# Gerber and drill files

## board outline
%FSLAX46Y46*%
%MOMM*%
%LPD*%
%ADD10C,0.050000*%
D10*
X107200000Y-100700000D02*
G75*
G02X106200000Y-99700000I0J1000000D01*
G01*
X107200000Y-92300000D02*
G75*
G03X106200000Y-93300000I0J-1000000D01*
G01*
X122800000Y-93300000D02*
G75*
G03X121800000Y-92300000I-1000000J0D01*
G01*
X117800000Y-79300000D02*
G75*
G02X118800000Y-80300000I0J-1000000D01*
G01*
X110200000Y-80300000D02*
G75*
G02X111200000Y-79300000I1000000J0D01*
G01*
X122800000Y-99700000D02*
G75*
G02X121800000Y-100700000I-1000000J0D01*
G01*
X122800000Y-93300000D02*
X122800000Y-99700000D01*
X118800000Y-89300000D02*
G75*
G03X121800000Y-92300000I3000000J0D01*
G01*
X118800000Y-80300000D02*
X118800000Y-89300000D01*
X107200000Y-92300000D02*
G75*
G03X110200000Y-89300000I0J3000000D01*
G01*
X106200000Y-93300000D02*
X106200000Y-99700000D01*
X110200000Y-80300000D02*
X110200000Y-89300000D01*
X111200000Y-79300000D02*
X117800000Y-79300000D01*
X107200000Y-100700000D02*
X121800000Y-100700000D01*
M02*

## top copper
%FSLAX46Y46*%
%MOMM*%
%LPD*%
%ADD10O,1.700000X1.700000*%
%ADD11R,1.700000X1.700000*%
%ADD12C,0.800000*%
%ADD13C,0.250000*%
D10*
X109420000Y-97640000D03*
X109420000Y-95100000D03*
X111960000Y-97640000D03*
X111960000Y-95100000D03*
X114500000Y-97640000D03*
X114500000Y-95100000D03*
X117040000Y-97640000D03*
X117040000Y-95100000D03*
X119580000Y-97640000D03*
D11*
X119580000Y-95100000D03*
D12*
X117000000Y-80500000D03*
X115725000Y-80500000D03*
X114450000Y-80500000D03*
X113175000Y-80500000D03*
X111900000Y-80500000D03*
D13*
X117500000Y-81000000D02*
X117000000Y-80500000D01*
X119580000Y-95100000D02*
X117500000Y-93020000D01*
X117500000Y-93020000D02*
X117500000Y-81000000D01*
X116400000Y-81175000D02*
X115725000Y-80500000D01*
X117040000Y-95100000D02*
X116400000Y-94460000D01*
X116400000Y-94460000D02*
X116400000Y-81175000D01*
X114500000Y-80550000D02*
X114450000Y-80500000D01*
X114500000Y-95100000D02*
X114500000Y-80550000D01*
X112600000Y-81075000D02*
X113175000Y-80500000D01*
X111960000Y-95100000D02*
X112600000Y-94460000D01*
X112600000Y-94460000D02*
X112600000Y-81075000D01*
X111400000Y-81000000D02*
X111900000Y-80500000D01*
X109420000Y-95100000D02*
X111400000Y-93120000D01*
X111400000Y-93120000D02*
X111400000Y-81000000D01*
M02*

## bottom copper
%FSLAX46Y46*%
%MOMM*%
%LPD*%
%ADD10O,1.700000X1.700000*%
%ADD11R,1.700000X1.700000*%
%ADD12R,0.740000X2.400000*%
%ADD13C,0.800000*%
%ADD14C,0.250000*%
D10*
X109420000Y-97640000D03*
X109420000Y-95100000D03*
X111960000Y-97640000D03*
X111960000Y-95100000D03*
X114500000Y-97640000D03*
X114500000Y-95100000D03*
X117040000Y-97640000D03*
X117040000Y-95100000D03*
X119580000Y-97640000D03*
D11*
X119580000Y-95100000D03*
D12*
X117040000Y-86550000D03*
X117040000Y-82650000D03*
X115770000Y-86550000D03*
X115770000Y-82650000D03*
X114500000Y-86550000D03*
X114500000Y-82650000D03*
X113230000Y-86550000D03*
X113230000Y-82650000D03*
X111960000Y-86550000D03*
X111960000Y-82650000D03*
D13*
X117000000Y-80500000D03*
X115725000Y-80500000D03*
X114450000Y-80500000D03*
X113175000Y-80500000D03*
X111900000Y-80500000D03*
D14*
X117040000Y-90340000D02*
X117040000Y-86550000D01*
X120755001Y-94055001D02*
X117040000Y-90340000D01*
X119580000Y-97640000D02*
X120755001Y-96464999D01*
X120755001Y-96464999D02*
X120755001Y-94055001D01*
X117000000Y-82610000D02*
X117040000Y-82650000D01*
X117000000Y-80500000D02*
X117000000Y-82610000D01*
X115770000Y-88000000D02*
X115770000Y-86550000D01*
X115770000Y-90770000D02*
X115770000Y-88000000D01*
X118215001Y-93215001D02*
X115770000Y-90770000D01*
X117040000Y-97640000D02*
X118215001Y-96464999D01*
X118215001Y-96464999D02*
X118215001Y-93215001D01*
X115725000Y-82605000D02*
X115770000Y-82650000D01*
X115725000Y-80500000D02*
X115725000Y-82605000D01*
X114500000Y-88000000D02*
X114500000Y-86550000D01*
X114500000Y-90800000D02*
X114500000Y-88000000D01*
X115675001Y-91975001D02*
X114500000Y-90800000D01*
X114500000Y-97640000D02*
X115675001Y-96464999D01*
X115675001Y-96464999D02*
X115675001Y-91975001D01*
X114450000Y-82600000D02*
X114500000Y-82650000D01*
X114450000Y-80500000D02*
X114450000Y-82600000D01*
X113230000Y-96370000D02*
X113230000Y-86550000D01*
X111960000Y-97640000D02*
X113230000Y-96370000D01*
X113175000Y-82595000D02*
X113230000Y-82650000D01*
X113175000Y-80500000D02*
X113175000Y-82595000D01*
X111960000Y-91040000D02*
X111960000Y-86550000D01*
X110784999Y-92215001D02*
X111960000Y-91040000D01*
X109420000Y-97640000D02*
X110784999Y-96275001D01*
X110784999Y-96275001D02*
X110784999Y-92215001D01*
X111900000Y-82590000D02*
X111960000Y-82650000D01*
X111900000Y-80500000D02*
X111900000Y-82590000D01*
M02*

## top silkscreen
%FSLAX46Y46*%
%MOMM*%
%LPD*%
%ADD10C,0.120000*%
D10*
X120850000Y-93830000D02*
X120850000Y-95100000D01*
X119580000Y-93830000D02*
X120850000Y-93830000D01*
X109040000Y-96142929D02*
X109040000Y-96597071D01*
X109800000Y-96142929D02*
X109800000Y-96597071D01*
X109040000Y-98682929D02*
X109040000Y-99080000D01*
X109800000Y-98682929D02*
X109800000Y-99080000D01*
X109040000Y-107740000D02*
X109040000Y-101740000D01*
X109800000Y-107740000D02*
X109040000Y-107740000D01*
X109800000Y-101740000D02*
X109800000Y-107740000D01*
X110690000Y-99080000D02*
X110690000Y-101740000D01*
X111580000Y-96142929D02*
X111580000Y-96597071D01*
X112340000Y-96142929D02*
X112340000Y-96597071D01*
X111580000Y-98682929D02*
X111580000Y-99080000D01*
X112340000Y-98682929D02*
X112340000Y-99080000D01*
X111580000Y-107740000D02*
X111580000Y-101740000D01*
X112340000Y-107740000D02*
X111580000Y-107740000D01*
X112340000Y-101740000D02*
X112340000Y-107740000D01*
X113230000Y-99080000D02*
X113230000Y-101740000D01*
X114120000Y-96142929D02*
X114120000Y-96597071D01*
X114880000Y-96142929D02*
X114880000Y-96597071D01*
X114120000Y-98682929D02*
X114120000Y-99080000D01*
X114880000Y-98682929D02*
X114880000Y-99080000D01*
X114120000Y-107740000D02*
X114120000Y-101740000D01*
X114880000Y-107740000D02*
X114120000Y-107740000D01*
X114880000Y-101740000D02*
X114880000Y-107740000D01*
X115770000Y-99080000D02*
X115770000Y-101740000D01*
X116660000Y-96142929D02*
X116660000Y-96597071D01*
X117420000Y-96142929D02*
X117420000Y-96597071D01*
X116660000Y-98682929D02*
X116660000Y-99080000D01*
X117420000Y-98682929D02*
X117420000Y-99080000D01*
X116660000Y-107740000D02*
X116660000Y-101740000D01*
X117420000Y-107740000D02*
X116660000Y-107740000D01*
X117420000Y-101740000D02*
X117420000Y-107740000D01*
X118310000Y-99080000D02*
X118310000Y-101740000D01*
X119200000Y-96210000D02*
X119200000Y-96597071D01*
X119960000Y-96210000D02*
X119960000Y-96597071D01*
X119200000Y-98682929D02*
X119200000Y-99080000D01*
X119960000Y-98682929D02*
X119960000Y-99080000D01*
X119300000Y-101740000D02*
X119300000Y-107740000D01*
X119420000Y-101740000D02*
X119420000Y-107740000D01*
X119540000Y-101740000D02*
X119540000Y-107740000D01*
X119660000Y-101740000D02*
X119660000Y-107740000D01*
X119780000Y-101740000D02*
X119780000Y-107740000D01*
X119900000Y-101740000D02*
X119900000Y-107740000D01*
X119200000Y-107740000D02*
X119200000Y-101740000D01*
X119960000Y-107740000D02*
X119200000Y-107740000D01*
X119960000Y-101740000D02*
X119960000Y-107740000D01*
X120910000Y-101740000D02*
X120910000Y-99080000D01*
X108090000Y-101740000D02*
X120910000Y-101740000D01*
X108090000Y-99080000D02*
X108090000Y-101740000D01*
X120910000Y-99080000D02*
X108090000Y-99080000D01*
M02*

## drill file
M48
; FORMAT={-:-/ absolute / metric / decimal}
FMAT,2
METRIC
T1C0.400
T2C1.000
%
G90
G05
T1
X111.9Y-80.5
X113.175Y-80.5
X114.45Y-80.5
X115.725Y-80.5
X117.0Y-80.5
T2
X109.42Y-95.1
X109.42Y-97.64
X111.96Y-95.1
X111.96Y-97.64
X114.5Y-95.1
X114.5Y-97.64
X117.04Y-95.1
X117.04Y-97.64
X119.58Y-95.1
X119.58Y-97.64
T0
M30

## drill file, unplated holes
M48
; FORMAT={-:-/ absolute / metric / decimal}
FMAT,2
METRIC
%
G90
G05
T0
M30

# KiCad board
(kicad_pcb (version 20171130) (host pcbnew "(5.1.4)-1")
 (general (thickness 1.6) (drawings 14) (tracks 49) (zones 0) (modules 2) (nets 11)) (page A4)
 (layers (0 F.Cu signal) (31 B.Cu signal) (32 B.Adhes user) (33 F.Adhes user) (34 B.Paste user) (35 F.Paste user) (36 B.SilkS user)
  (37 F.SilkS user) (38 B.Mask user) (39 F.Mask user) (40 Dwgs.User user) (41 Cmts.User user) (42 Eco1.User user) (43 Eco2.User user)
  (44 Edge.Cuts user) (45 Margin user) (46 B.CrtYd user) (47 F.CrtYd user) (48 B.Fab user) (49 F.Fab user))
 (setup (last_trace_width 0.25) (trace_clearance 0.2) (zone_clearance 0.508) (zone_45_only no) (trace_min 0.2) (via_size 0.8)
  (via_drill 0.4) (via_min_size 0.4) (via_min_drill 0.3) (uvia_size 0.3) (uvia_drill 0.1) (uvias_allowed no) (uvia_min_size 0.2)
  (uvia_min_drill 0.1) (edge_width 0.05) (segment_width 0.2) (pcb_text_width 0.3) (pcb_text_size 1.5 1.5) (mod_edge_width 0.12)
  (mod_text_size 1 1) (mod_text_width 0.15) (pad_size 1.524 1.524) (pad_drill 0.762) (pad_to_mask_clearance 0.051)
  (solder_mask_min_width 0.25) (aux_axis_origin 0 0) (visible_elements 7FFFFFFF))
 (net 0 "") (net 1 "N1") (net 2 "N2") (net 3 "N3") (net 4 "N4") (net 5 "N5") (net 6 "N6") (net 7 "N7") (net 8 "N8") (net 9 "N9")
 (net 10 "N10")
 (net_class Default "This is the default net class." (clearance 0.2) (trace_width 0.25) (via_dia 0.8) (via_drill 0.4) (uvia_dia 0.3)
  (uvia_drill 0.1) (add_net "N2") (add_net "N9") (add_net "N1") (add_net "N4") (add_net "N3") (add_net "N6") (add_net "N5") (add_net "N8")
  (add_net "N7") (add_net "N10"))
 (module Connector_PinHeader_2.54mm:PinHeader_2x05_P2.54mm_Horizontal (layer F.Cu) (at 119.58 95.1 270)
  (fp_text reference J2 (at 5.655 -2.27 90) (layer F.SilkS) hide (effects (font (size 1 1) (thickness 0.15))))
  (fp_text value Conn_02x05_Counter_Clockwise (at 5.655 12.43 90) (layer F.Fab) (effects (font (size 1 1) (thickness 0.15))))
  (fp_line (start -1.27 -1.27) (end 0 -1.27) (layer F.SilkS) (width 0.12))
  (fp_line (start -1.27 0) (end -1.27 -1.27) (layer F.SilkS) (width 0.12))
  (fp_line (start 1.042929 10.54) (end 1.497071 10.54) (layer F.SilkS) (width 0.12))
  (fp_line (start 1.042929 9.78) (end 1.497071 9.78) (layer F.SilkS) (width 0.12))
  (fp_line (start 3.582929 10.54) (end 3.98 10.54) (layer F.SilkS) (width 0.12))
  (fp_line (start 3.582929 9.78) (end 3.98 9.78) (layer F.SilkS) (width 0.12))
  (fp_line (start 12.64 10.54) (end 6.64 10.54) (layer F.SilkS) (width 0.12))
  (fp_line (start 12.64 9.78) (end 12.64 10.54) (layer F.SilkS) (width 0.12))
  (fp_line (start 6.64 9.78) (end 12.64 9.78) (layer F.SilkS) (width 0.12))
  (fp_line (start 3.98 8.89) (end 6.64 8.89) (layer F.SilkS) (width 0.12))
  (fp_line (start 1.042929 8) (end 1.497071 8) (layer F.SilkS) (width 0.12))
  (fp_line (start 1.042929 7.24) (end 1.497071 7.24) (layer F.SilkS) (width 0.12))
  (fp_line (start 3.582929 8) (end 3.98 8) (layer F.SilkS) (width 0.12))
  (fp_line (start 3.582929 7.24) (end 3.98 7.24) (layer F.SilkS) (width 0.12))
  (fp_line (start 12.64 8) (end 6.64 8) (layer F.SilkS) (width 0.12))
  (fp_line (start 12.64 7.24) (end 12.64 8) (layer F.SilkS) (width 0.12))
  (fp_line (start 6.64 7.24) (end 12.64 7.24) (layer F.SilkS) (width 0.12))
  (fp_line (start 3.98 6.35) (end 6.64 6.35) (layer F.SilkS) (width 0.12))
  (fp_line (start 1.042929 5.46) (end 1.497071 5.46) (layer F.SilkS) (width 0.12))
  (fp_line (start 1.042929 4.7) (end 1.497071 4.7) (layer F.SilkS) (width 0.12))
  (fp_line (start 3.582929 5.46) (end 3.98 5.46) (layer F.SilkS) (width 0.12))
  (fp_line (start 3.582929 4.7) (end 3.98 4.7) (layer F.SilkS) (width 0.12))
  (fp_line (start 12.64 5.46) (end 6.64 5.46) (layer F.SilkS) (width 0.12))
  (fp_line (start 12.64 4.7) (end 12.64 5.46) (layer F.SilkS) (width 0.12))
  (fp_line (start 6.64 4.7) (end 12.64 4.7) (layer F.SilkS) (width 0.12))
  (fp_line (start 3.98 3.81) (end 6.64 3.81) (layer F.SilkS) (width 0.12))
  (fp_line (start 1.042929 2.92) (end 1.497071 2.92) (layer F.SilkS) (width 0.12))
  (fp_line (start 1.042929 2.16) (end 1.497071 2.16) (layer F.SilkS) (width 0.12))
  (fp_line (start 3.582929 2.92) (end 3.98 2.92) (layer F.SilkS) (width 0.12))
  (fp_line (start 3.582929 2.16) (end 3.98 2.16) (layer F.SilkS) (width 0.12))
  (fp_line (start 12.64 2.92) (end 6.64 2.92) (layer F.SilkS) (width 0.12))
  (fp_line (start 12.64 2.16) (end 12.64 2.92) (layer F.SilkS) (width 0.12))
  (fp_line (start 6.64 2.16) (end 12.64 2.16) (layer F.SilkS) (width 0.12))
  (fp_line (start 3.98 1.27) (end 6.64 1.27) (layer F.SilkS) (width 0.12))
  (fp_line (start 1.11 0.38) (end 1.497071 0.38) (layer F.SilkS) (width 0.12))
  (fp_line (start 1.11 -0.38) (end 1.497071 -0.38) (layer F.SilkS) (width 0.12))
  (fp_line (start 3.582929 0.38) (end 3.98 0.38) (layer F.SilkS) (width 0.12))
  (fp_line (start 3.582929 -0.38) (end 3.98 -0.38) (layer F.SilkS) (width 0.12))
  (fp_line (start 6.64 0.28) (end 12.64 0.28) (layer F.SilkS) (width 0.12))
  (fp_line (start 6.64 0.16) (end 12.64 0.16) (layer F.SilkS) (width 0.12))
  (fp_line (start 6.64 0.04) (end 12.64 0.04) (layer F.SilkS) (width 0.12))
  (fp_line (start 6.64 -0.08) (end 12.64 -0.08) (layer F.SilkS) (width 0.12))
  (fp_line (start 6.64 -0.2) (end 12.64 -0.2) (layer F.SilkS) (width 0.12))
  (fp_line (start 6.64 -0.32) (end 12.64 -0.32) (layer F.SilkS) (width 0.12))
  (fp_line (start 12.64 0.38) (end 6.64 0.38) (layer F.SilkS) (width 0.12))
  (fp_line (start 12.64 -0.38) (end 12.64 0.38) (layer F.SilkS) (width 0.12))
  (fp_line (start 6.64 -0.38) (end 12.64 -0.38) (layer F.SilkS) (width 0.12))
  (fp_line (start 6.64 -1.33) (end 3.98 -1.33) (layer F.SilkS) (width 0.12))
  (fp_line (start 6.64 11.49) (end 6.64 -1.33) (layer F.SilkS) (width 0.12))
  (fp_line (start 3.98 11.49) (end 6.64 11.49) (layer F.SilkS) (width 0.12))
  (fp_line (start 3.98 -1.33) (end 3.98 11.49) (layer F.SilkS) (width 0.12))
  (pad 10 thru_hole oval (at 2.54 10.16 270) (size 1.7 1.7) (drill 1) (layers *.Cu *.Mask) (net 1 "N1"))
  (pad 9 thru_hole oval (at 0 10.16 270) (size 1.7 1.7) (drill 1) (layers *.Cu *.Mask) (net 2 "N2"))
  (pad 8 thru_hole oval (at 2.54 7.62 270) (size 1.7 1.7) (drill 1) (layers *.Cu *.Mask) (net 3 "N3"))
  (pad 7 thru_hole oval (at 0 7.62 270) (size 1.7 1.7) (drill 1) (layers *.Cu *.Mask) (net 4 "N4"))
  (pad 6 thru_hole oval (at 2.54 5.08 270) (size 1.7 1.7) (drill 1) (layers *.Cu *.Mask) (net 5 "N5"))
  (pad 5 thru_hole oval (at 0 5.08 270) (size 1.7 1.7) (drill 1) (layers *.Cu *.Mask) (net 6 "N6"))
  (pad 4 thru_hole oval (at 2.54 2.54 270) (size 1.7 1.7) (drill 1) (layers *.Cu *.Mask) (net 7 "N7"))
  (pad 3 thru_hole oval (at 0 2.54 270) (size 1.7 1.7) (drill 1) (layers *.Cu *.Mask) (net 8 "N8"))
  (pad 2 thru_hole oval (at 2.54 0 270) (size 1.7 1.7) (drill 1) (layers *.Cu *.Mask) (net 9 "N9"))
  (pad 1 thru_hole rect (at 0 0 270) (size 1.7 1.7) (drill 1) (layers *.Cu *.Mask) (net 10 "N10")))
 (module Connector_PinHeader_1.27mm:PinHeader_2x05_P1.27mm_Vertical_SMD (layer B.Cu) (at 114.5 84.6 270)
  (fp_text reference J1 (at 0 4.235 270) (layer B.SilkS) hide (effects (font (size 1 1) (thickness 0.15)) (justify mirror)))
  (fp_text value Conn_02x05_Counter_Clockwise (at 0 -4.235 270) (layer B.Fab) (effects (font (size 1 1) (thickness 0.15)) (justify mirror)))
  (pad 10 smd rect (at 1.95 -2.54 270) (size 2.4 0.74) (layers B.Cu B.Paste B.Mask) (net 9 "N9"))
  (pad 9 smd rect (at -1.95 -2.54 270) (size 2.4 0.74) (layers B.Cu B.Paste B.Mask) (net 10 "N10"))
  (pad 8 smd rect (at 1.95 -1.27 270) (size 2.4 0.74) (layers B.Cu B.Paste B.Mask) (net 7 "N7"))
  (pad 7 smd rect (at -1.95 -1.27 270) (size 2.4 0.74) (layers B.Cu B.Paste B.Mask) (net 8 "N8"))
  (pad 6 smd rect (at 1.95 0 270) (size 2.4 0.74) (layers B.Cu B.Paste B.Mask) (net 5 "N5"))
  (pad 5 smd rect (at -1.95 0 270) (size 2.4 0.74) (layers B.Cu B.Paste B.Mask) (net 6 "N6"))
  (pad 4 smd rect (at 1.95 1.27 270) (size 2.4 0.74) (layers B.Cu B.Paste B.Mask) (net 3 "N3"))
  (pad 3 smd rect (at -1.95 1.27 270) (size 2.4 0.74) (layers B.Cu B.Paste B.Mask) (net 4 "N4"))
  (pad 2 smd rect (at 1.95 2.54 270) (size 2.4 0.74) (layers B.Cu B.Paste B.Mask) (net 1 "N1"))
  (pad 1 smd rect (at -1.95 2.54 270) (size 2.4 0.74) (layers B.Cu B.Paste B.Mask) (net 2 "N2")))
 (gr_arc (start 107.2 99.7) (end 106.2 99.7) (angle -90) (layer Edge.Cuts) (width 0.05))
 (gr_arc (start 107.2 93.3) (end 106.2 93.3) (angle 90) (layer Edge.Cuts) (width 0.05))
 (gr_arc (start 121.8 93.3) (end 121.8 92.3) (angle 90) (layer Edge.Cuts) (width 0.05))
 (gr_arc (start 117.8 80.3) (end 118.8 80.3) (angle -90) (layer Edge.Cuts) (width 0.05))
 (gr_arc (start 111.2 80.3) (end 111.2 79.3) (angle -90) (layer Edge.Cuts) (width 0.05))
 (gr_arc (start 121.8 99.7) (end 121.8 100.7) (angle -90) (layer Edge.Cuts) (width 0.05))
 (gr_line (start 122.8 93.3) (end 122.8 99.7) (layer Edge.Cuts) (width 0.05))
 (gr_arc (start 121.8 89.3) (end 121.8 92.3) (angle 90) (layer Edge.Cuts) (width 0.05))
 (gr_line (start 118.8 80.3) (end 118.8 89.3) (layer Edge.Cuts) (width 0.05))
 (gr_arc (start 107.2 89.3) (end 110.2 89.3) (angle 90) (layer Edge.Cuts) (width 0.05))
 (gr_line (start 106.2 93.3) (end 106.2 99.7) (layer Edge.Cuts) (width 0.05))
 (gr_line (start 110.2 80.3) (end 110.2 89.3) (layer Edge.Cuts) (width 0.05))
 (gr_line (start 111.2 79.3) (end 117.8 79.3) (layer Edge.Cuts) (width 0.05))
 (gr_line (start 107.2 100.7) (end 121.8 100.7) (layer Edge.Cuts) (width 0.05))
 (segment (start 117.04 90.34) (end 117.04 86.55) (width 0.25) (layer B.Cu) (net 9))
 (segment (start 120.755001 94.055001) (end 117.04 90.34) (width 0.25) (layer B.Cu) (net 9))
 (segment (start 119.58 97.64) (end 120.755001 96.464999) (width 0.25) (layer B.Cu) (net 9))
 (segment (start 120.755001 96.464999) (end 120.755001 94.055001) (width 0.25) (layer B.Cu) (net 9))
 (via (at 117 80.5) (size 0.8) (drill 0.4) (layers F.Cu B.Cu) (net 10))
 (segment (start 117 82.61) (end 117.04 82.65) (width 0.25) (layer B.Cu) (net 10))
 (segment (start 117 80.5) (end 117 82.61) (width 0.25) (layer B.Cu) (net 10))
 (segment (start 117.5 81) (end 117 80.5) (width 0.25) (layer F.Cu) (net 10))
 (segment (start 119.58 95.1) (end 117.5 93.02) (width 0.25) (layer F.Cu) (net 10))
 (segment (start 117.5 93.02) (end 117.5 81) (width 0.25) (layer F.Cu) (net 10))
 (segment (start 115.77 88) (end 115.77 86.55) (width 0.25) (layer B.Cu) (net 7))
 (segment (start 115.77 90.77) (end 115.77 88) (width 0.25) (layer B.Cu) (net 7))
 (segment (start 118.215001 93.215001) (end 115.77 90.77) (width 0.25) (layer B.Cu) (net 7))
 (segment (start 117.04 97.64) (end 118.215001 96.464999) (width 0.25) (layer B.Cu) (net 7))
 (segment (start 118.215001 96.464999) (end 118.215001 93.215001) (width 0.25) (layer B.Cu) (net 7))
 (via (at 115.725 80.5) (size 0.8) (drill 0.4) (layers F.Cu B.Cu) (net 8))
 (segment (start 115.725 82.605) (end 115.77 82.65) (width 0.25) (layer B.Cu) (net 8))
 (segment (start 115.725 80.5) (end 115.725 82.605) (width 0.25) (layer B.Cu) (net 8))
 (segment (start 116.4 81.175) (end 115.725 80.5) (width 0.25) (layer F.Cu) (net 8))
 (segment (start 117.04 95.1) (end 116.4 94.46) (width 0.25) (layer F.Cu) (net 8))
 (segment (start 116.4 94.46) (end 116.4 81.175) (width 0.25) (layer F.Cu) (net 8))
 (segment (start 114.5 88) (end 114.5 86.55) (width 0.25) (layer B.Cu) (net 5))
 (segment (start 114.5 90.8) (end 114.5 88) (width 0.25) (layer B.Cu) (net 5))
 (segment (start 115.675001 91.975001) (end 114.5 90.8) (width 0.25) (layer B.Cu) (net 5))
 (segment (start 114.5 97.64) (end 115.675001 96.464999) (width 0.25) (layer B.Cu) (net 5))
 (segment (start 115.675001 96.464999) (end 115.675001 91.975001) (width 0.25) (layer B.Cu) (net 5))
 (via (at 114.45 80.5) (size 0.8) (drill 0.4) (layers F.Cu B.Cu) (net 6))
 (segment (start 114.5 80.55) (end 114.45 80.5) (width 0.25) (layer F.Cu) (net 6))
 (segment (start 114.5 95.1) (end 114.5 80.55) (width 0.25) (layer F.Cu) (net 6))
 (segment (start 114.45 82.6) (end 114.5 82.65) (width 0.25) (layer B.Cu) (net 6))
 (segment (start 114.45 80.5) (end 114.45 82.6) (width 0.25) (layer B.Cu) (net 6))
 (segment (start 113.23 96.37) (end 113.23 86.55) (width 0.25) (layer B.Cu) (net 3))
 (segment (start 111.96 97.64) (end 113.23 96.37) (width 0.25) (layer B.Cu) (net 3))
 (via (at 113.175 80.5) (size 0.8) (drill 0.4) (layers F.Cu B.Cu) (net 4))
 (segment (start 113.175 82.595) (end 113.23 82.65) (width 0.25) (layer B.Cu) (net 4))
 (segment (start 113.175 80.5) (end 113.175 82.595) (width 0.25) (layer B.Cu) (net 4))
 (segment (start 112.6 81.075) (end 113.175 80.5) (width 0.25) (layer F.Cu) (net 4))
 (segment (start 111.96 95.1) (end 112.6 94.46) (width 0.25) (layer F.Cu) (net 4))
 (segment (start 112.6 94.46) (end 112.6 81.075) (width 0.25) (layer F.Cu) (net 4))
 (segment (start 111.96 91.04) (end 111.96 86.55) (width 0.25) (layer B.Cu) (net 1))
 (segment (start 110.784999 92.215001) (end 111.96 91.04) (width 0.25) (layer B.Cu) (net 1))
 (segment (start 109.42 97.64) (end 110.784999 96.275001) (width 0.25) (layer B.Cu) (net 1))
 (segment (start 110.784999 96.275001) (end 110.784999 92.215001) (width 0.25) (layer B.Cu) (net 1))
 (via (at 111.9 80.5) (size 0.8) (drill 0.4) (layers F.Cu B.Cu) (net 2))
 (segment (start 111.9 82.59) (end 111.96 82.65) (width 0.25) (layer B.Cu) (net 2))
 (segment (start 111.9 80.5) (end 111.9 82.59) (width 0.25) (layer B.Cu) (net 2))
 (segment (start 111.4 81) (end 111.9 80.5) (width 0.25) (layer F.Cu) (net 2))
 (segment (start 109.42 95.1) (end 111.4 93.12) (width 0.25) (layer F.Cu) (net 2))
 (segment (start 111.4 93.12) (end 111.4 81) (width 0.25) (layer F.Cu) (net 2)))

